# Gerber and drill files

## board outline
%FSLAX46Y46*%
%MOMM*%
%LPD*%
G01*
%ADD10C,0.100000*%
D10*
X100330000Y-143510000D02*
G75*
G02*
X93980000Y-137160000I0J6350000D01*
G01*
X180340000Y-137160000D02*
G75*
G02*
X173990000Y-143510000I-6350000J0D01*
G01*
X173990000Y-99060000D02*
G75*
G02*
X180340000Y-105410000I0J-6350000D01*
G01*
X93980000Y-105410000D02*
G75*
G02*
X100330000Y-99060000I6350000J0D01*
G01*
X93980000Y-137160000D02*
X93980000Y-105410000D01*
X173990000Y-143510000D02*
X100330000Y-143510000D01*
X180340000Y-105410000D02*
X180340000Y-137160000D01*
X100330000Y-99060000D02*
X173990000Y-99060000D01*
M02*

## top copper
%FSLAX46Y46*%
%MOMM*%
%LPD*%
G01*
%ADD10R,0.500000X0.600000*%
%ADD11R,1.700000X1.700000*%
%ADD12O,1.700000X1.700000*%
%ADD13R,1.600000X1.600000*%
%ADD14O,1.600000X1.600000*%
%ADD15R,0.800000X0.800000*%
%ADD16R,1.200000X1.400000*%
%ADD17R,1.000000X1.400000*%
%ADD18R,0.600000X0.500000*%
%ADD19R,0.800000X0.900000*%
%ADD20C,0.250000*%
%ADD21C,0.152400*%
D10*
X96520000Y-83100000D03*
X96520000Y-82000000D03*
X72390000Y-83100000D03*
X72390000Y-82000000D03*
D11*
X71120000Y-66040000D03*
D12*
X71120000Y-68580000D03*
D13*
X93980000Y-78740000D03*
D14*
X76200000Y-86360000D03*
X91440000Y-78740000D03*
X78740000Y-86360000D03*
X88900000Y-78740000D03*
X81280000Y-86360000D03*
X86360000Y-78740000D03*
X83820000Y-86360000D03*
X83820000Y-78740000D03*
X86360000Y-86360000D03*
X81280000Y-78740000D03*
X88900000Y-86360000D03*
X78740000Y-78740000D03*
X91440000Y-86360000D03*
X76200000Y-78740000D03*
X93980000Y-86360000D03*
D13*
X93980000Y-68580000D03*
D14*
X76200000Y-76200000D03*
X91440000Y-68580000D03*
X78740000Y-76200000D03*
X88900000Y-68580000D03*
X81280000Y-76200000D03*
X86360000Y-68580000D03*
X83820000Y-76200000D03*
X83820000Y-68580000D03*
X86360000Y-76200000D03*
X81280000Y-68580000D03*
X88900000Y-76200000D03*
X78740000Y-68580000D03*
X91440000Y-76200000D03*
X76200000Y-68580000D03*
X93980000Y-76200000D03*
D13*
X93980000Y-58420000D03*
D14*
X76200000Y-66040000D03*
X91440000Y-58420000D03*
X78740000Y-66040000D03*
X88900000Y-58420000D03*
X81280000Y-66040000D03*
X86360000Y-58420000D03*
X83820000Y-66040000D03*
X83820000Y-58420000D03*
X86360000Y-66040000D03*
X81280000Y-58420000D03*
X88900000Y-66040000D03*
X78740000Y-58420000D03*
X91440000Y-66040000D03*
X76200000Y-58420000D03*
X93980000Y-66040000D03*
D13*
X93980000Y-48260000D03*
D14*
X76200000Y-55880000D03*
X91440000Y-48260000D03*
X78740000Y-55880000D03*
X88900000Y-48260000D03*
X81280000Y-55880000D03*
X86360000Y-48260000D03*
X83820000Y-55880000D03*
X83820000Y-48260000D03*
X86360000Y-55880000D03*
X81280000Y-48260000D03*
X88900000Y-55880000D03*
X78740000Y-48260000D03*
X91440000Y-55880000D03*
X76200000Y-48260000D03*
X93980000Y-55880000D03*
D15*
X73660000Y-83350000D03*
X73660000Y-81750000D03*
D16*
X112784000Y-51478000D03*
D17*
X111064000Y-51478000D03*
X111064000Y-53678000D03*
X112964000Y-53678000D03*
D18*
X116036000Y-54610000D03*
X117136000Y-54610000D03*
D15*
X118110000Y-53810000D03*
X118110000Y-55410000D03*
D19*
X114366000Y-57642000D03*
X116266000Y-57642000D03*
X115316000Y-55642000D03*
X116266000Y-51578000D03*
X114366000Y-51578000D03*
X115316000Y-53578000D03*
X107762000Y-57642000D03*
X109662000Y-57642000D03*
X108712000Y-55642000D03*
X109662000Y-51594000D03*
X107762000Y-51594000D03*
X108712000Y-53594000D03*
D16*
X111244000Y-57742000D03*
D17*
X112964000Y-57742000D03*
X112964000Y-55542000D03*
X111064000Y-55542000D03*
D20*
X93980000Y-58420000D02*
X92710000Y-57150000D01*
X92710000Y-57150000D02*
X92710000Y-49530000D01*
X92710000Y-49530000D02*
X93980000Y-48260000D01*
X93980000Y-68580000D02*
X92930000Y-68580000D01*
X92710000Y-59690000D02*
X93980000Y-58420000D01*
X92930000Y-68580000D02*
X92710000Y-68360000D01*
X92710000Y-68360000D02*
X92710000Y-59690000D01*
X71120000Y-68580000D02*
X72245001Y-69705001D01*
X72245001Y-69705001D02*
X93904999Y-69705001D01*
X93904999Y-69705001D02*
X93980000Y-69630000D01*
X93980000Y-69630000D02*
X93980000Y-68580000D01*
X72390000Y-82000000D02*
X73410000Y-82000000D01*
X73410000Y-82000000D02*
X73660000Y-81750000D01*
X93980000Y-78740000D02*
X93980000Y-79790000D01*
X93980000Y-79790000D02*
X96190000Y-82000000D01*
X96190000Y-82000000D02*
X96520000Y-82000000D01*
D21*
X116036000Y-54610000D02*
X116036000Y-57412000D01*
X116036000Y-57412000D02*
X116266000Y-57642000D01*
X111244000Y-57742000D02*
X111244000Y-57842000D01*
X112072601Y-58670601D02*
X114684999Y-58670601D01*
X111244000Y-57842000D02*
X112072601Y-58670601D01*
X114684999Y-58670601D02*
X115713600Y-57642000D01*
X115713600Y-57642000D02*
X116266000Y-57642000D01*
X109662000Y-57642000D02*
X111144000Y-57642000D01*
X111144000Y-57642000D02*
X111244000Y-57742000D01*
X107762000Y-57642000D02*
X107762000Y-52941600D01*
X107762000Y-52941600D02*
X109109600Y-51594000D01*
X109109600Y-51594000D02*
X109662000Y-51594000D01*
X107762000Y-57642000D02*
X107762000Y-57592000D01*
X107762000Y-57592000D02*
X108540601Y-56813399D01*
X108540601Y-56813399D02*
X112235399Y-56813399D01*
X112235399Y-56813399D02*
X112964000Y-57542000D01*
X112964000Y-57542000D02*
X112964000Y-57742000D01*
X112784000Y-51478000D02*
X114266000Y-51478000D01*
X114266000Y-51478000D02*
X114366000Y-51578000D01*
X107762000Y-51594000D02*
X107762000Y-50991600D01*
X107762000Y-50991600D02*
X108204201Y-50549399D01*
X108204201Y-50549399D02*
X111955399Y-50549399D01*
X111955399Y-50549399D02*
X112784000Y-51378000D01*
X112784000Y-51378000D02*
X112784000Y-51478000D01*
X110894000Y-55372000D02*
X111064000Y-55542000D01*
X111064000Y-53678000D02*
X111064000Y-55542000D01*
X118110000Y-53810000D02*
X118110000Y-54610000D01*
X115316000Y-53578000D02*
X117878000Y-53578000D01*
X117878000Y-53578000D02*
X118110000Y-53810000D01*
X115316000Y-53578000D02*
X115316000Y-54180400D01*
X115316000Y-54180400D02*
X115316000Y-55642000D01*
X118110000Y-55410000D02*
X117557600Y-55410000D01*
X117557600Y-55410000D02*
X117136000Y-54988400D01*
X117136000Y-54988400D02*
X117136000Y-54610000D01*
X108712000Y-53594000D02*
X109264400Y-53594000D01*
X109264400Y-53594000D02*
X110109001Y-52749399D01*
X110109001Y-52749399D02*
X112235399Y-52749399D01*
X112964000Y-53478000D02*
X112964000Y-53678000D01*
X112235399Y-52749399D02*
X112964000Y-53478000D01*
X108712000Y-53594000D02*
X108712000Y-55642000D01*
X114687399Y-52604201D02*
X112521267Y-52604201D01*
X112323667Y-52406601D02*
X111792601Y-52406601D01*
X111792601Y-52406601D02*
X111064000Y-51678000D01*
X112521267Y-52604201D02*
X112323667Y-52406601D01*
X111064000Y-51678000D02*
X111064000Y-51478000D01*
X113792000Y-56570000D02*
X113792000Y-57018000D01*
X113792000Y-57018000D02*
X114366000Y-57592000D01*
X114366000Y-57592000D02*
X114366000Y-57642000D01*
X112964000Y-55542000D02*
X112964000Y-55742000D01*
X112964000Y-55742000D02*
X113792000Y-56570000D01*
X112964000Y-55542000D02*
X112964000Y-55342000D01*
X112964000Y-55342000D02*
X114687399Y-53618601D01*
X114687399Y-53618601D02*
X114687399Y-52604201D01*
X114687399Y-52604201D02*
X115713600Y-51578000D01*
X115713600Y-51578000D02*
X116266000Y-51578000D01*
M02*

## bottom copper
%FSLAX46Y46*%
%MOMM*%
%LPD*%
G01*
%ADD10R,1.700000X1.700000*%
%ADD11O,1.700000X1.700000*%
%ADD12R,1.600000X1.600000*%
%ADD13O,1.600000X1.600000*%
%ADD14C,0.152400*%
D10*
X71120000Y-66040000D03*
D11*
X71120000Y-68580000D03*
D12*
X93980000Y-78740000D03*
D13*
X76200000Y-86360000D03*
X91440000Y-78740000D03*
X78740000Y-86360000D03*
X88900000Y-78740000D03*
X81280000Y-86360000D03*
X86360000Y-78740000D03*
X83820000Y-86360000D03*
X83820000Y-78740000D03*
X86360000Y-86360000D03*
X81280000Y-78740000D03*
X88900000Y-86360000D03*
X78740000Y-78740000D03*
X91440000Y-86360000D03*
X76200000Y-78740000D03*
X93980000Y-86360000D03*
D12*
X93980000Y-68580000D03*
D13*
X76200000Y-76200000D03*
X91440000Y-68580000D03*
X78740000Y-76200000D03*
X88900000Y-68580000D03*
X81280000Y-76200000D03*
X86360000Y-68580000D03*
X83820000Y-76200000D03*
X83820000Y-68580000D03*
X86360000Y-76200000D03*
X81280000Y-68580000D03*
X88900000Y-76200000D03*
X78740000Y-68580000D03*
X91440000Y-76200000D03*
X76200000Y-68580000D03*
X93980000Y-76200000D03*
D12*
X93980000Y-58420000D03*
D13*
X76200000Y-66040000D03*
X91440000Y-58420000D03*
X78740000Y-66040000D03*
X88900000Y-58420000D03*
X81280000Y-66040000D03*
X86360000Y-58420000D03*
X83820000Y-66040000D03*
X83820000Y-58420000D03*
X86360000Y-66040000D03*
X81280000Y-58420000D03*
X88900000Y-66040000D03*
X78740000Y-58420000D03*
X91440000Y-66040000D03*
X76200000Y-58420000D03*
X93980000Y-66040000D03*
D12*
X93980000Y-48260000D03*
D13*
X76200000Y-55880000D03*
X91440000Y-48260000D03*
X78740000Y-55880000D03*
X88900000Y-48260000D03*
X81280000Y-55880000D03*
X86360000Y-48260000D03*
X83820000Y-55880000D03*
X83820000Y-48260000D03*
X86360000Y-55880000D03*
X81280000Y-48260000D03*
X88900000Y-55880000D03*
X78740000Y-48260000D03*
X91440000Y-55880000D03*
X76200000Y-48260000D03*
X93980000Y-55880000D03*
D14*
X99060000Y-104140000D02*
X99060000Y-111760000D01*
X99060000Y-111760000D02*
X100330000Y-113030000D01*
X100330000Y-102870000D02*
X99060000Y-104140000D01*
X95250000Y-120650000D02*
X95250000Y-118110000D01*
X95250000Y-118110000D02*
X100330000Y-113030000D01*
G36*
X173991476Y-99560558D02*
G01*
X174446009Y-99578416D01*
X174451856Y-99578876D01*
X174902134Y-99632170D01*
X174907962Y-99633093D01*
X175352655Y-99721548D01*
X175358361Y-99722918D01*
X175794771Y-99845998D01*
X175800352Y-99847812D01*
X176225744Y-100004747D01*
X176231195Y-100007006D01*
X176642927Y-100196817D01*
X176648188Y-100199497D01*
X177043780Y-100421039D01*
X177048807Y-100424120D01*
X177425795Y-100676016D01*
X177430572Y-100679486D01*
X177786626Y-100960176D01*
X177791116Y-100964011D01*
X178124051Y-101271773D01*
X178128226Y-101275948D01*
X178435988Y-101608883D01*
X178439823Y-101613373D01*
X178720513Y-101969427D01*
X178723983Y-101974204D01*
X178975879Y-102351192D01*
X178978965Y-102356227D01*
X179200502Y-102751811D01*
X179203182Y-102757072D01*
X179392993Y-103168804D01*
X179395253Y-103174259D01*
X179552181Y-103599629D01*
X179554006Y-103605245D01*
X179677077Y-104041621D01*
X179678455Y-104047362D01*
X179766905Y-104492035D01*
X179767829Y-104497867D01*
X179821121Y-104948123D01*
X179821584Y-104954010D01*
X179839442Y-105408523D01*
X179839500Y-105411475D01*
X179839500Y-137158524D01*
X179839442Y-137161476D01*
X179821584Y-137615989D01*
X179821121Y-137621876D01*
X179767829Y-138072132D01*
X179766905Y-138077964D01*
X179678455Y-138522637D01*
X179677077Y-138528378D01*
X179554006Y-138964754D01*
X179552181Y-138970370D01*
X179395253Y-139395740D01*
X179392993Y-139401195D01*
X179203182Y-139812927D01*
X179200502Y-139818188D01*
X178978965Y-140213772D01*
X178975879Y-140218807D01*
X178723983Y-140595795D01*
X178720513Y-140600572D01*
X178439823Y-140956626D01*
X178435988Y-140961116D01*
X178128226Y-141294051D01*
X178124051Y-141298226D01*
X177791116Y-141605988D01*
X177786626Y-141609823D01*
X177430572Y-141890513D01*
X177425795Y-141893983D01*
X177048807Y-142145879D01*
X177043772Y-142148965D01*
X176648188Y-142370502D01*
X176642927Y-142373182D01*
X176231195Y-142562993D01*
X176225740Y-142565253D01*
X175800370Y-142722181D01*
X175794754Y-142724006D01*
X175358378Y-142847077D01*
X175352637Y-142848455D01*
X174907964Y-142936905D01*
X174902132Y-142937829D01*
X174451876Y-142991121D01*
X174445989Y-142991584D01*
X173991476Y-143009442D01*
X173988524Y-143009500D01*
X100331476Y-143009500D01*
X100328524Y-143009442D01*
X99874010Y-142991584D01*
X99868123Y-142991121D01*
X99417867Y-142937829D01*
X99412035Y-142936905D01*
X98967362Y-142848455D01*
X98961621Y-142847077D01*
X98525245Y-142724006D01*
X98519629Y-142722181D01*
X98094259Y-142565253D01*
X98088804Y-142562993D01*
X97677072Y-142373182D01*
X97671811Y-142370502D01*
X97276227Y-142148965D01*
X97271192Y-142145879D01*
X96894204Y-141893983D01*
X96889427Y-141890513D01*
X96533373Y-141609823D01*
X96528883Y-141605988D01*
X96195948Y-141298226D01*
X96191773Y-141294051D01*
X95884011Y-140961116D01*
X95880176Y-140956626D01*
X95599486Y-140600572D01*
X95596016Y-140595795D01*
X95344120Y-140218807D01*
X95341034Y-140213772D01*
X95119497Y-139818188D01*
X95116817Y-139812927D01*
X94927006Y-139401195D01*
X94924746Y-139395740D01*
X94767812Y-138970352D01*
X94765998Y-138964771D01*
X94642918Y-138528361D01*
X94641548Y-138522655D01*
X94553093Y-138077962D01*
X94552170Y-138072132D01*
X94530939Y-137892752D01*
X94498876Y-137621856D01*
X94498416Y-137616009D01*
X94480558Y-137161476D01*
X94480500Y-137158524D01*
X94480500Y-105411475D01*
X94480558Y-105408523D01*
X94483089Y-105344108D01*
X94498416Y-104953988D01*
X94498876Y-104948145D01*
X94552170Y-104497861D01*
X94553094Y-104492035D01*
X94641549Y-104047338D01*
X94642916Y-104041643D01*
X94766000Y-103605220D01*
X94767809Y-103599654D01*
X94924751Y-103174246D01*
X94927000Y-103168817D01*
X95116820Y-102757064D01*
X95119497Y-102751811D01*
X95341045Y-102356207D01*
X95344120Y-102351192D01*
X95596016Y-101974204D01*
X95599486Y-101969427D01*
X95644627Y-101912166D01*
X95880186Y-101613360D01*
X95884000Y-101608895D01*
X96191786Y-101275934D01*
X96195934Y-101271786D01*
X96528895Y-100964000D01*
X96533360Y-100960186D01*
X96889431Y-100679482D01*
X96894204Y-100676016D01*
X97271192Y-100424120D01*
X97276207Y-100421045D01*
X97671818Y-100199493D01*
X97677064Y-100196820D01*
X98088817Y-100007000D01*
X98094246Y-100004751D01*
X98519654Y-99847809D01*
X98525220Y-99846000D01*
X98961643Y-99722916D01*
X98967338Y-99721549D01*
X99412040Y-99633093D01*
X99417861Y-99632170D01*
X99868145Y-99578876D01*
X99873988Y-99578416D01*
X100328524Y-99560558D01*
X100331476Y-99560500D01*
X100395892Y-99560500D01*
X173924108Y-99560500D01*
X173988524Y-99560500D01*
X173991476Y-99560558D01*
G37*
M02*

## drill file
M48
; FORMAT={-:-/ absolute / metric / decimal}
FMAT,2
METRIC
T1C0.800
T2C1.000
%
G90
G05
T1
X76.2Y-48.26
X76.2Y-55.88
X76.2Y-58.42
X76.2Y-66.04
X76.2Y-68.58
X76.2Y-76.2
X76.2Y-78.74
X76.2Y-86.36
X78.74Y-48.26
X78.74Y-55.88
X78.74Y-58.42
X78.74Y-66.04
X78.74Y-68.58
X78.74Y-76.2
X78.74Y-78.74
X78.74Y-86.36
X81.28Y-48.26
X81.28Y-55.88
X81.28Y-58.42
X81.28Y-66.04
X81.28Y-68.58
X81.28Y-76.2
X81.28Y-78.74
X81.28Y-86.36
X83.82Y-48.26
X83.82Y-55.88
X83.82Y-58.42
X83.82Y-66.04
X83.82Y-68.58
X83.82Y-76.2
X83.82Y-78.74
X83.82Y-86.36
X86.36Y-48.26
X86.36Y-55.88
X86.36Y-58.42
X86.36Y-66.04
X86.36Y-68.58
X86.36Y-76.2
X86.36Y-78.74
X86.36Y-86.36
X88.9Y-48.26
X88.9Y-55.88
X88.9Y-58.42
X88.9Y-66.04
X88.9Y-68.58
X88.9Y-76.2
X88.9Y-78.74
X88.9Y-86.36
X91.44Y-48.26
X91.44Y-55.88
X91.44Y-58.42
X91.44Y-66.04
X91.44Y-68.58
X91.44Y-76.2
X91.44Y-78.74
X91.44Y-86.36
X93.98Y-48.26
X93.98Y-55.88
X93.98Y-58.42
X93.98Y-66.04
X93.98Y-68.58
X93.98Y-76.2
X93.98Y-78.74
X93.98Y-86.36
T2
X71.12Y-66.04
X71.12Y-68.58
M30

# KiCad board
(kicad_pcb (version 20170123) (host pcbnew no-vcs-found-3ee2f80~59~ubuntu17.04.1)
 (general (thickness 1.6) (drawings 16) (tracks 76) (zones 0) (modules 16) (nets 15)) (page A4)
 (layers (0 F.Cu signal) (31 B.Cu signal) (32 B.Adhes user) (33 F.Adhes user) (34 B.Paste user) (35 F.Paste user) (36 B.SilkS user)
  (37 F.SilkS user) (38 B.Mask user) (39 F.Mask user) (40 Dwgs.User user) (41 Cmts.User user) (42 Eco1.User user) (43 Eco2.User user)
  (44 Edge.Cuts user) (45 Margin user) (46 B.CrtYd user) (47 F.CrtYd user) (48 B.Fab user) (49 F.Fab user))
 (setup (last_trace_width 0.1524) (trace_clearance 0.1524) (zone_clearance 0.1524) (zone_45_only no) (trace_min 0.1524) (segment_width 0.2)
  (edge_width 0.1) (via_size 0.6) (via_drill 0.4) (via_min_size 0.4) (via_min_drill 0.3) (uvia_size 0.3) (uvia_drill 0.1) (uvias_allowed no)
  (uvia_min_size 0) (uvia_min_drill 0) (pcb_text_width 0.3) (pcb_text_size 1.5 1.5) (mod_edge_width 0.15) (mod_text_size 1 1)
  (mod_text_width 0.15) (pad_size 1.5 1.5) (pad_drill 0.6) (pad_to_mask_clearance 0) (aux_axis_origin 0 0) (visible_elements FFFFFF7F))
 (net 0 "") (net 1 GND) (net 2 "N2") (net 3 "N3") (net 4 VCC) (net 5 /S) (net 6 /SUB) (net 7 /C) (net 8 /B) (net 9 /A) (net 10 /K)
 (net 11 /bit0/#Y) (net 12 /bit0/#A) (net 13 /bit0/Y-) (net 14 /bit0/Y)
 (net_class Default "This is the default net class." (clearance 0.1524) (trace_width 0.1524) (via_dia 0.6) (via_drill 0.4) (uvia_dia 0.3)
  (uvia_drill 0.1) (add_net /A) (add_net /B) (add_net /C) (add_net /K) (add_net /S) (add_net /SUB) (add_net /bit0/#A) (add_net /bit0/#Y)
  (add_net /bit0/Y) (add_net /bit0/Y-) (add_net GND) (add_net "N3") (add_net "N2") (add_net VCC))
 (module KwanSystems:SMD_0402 (layer F.Cu) (at 96.52 82.55 270)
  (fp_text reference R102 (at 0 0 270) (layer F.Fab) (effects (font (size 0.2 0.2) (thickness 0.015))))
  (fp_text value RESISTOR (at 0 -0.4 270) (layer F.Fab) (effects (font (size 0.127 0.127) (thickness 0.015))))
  (pad 2 smd rect (at 0.55 0 270) (size 0.6 0.5) (layers F.Cu F.Paste F.Mask) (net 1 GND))
  (pad 1 smd rect (at -0.55 0 270) (size 0.6 0.5) (layers F.Cu F.Paste F.Mask) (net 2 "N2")))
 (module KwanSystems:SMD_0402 (layer F.Cu) (at 72.39 82.55 270)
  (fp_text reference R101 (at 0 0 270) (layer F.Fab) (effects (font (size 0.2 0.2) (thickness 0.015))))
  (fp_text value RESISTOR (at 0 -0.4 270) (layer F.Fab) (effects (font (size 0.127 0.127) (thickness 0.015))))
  (pad 2 smd rect (at 0.55 0 270) (size 0.6 0.5) (layers F.Cu F.Paste F.Mask) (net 1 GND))
  (pad 1 smd rect (at -0.55 0 270) (size 0.6 0.5) (layers F.Cu F.Paste F.Mask) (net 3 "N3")))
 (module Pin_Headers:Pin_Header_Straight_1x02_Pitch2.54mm (layer F.Cu) (at 71.12 66.04)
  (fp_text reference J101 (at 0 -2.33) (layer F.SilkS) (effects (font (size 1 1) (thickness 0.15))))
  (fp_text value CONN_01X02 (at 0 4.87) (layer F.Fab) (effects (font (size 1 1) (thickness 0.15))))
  (pad 1 thru_hole rect (at 0 0) (size 1.7 1.7) (drill 1) (layers *.Cu *.Mask) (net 1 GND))
  (pad 2 thru_hole oval (at 0 2.54) (size 1.7 1.7) (drill 1) (layers *.Cu *.Mask) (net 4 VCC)))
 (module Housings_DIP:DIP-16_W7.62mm (layer F.Cu) (at 93.98 78.74 270)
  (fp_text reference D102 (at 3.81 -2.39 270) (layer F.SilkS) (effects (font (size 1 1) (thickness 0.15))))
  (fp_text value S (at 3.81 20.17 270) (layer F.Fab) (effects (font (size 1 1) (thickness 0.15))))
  (pad 1 thru_hole rect (at 0 0 270) (size 1.6 1.6) (drill 0.8) (layers *.Cu *.Mask) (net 2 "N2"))
  (pad 9 thru_hole oval (at 7.62 17.78 270) (size 1.6 1.6) (drill 0.8) (layers *.Cu *.Mask))
  (pad 2 thru_hole oval (at 0 2.54 270) (size 1.6 1.6) (drill 0.8) (layers *.Cu *.Mask))
  (pad 10 thru_hole oval (at 7.62 15.24 270) (size 1.6 1.6) (drill 0.8) (layers *.Cu *.Mask))
  (pad 3 thru_hole oval (at 0 5.08 270) (size 1.6 1.6) (drill 0.8) (layers *.Cu *.Mask))
  (pad 11 thru_hole oval (at 7.62 12.7 270) (size 1.6 1.6) (drill 0.8) (layers *.Cu *.Mask))
  (pad 4 thru_hole oval (at 0 7.62 270) (size 1.6 1.6) (drill 0.8) (layers *.Cu *.Mask))
  (pad 12 thru_hole oval (at 7.62 10.16 270) (size 1.6 1.6) (drill 0.8) (layers *.Cu *.Mask))
  (pad 5 thru_hole oval (at 0 10.16 270) (size 1.6 1.6) (drill 0.8) (layers *.Cu *.Mask))
  (pad 13 thru_hole oval (at 7.62 7.62 270) (size 1.6 1.6) (drill 0.8) (layers *.Cu *.Mask))
  (pad 6 thru_hole oval (at 0 12.7 270) (size 1.6 1.6) (drill 0.8) (layers *.Cu *.Mask))
  (pad 14 thru_hole oval (at 7.62 5.08 270) (size 1.6 1.6) (drill 0.8) (layers *.Cu *.Mask))
  (pad 7 thru_hole oval (at 0 15.24 270) (size 1.6 1.6) (drill 0.8) (layers *.Cu *.Mask))
  (pad 15 thru_hole oval (at 7.62 2.54 270) (size 1.6 1.6) (drill 0.8) (layers *.Cu *.Mask))
  (pad 8 thru_hole oval (at 0 17.78 270) (size 1.6 1.6) (drill 0.8) (layers *.Cu *.Mask))
  (pad 16 thru_hole oval (at 7.62 0 270) (size 1.6 1.6) (drill 0.8) (layers *.Cu *.Mask) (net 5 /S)))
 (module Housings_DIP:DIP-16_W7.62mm (layer F.Cu) (at 93.98 68.58 270)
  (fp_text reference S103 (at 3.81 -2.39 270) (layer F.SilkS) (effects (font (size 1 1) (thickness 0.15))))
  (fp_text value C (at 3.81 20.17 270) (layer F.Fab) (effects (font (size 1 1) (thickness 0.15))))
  (pad 1 thru_hole rect (at 0 0 270) (size 1.6 1.6) (drill 0.8) (layers *.Cu *.Mask) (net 4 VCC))
  (pad 9 thru_hole oval (at 7.62 17.78 270) (size 1.6 1.6) (drill 0.8) (layers *.Cu *.Mask))
  (pad 2 thru_hole oval (at 0 2.54 270) (size 1.6 1.6) (drill 0.8) (layers *.Cu *.Mask))
  (pad 10 thru_hole oval (at 7.62 15.24 270) (size 1.6 1.6) (drill 0.8) (layers *.Cu *.Mask))
  (pad 3 thru_hole oval (at 0 5.08 270) (size 1.6 1.6) (drill 0.8) (layers *.Cu *.Mask))
  (pad 11 thru_hole oval (at 7.62 12.7 270) (size 1.6 1.6) (drill 0.8) (layers *.Cu *.Mask))
  (pad 4 thru_hole oval (at 0 7.62 270) (size 1.6 1.6) (drill 0.8) (layers *.Cu *.Mask))
  (pad 12 thru_hole oval (at 7.62 10.16 270) (size 1.6 1.6) (drill 0.8) (layers *.Cu *.Mask))
  (pad 5 thru_hole oval (at 0 10.16 270) (size 1.6 1.6) (drill 0.8) (layers *.Cu *.Mask))
  (pad 13 thru_hole oval (at 7.62 7.62 270) (size 1.6 1.6) (drill 0.8) (layers *.Cu *.Mask))
  (pad 6 thru_hole oval (at 0 12.7 270) (size 1.6 1.6) (drill 0.8) (layers *.Cu *.Mask))
  (pad 14 thru_hole oval (at 7.62 5.08 270) (size 1.6 1.6) (drill 0.8) (layers *.Cu *.Mask))
  (pad 7 thru_hole oval (at 0 15.24 270) (size 1.6 1.6) (drill 0.8) (layers *.Cu *.Mask))
  (pad 15 thru_hole oval (at 7.62 2.54 270) (size 1.6 1.6) (drill 0.8) (layers *.Cu *.Mask) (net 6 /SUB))
  (pad 8 thru_hole oval (at 0 17.78 270) (size 1.6 1.6) (drill 0.8) (layers *.Cu *.Mask) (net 1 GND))
  (pad 16 thru_hole oval (at 7.62 0 270) (size 1.6 1.6) (drill 0.8) (layers *.Cu *.Mask) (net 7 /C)))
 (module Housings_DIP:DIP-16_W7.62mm (layer F.Cu) (at 93.98 58.42 270)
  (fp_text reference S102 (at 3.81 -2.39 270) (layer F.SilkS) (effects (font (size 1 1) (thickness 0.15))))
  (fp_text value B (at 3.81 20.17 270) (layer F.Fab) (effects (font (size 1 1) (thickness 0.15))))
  (pad 1 thru_hole rect (at 0 0 270) (size 1.6 1.6) (drill 0.8) (layers *.Cu *.Mask) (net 4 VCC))
  (pad 9 thru_hole oval (at 7.62 17.78 270) (size 1.6 1.6) (drill 0.8) (layers *.Cu *.Mask))
  (pad 2 thru_hole oval (at 0 2.54 270) (size 1.6 1.6) (drill 0.8) (layers *.Cu *.Mask))
  (pad 10 thru_hole oval (at 7.62 15.24 270) (size 1.6 1.6) (drill 0.8) (layers *.Cu *.Mask))
  (pad 3 thru_hole oval (at 0 5.08 270) (size 1.6 1.6) (drill 0.8) (layers *.Cu *.Mask))
  (pad 11 thru_hole oval (at 7.62 12.7 270) (size 1.6 1.6) (drill 0.8) (layers *.Cu *.Mask))
  (pad 4 thru_hole oval (at 0 7.62 270) (size 1.6 1.6) (drill 0.8) (layers *.Cu *.Mask))
  (pad 12 thru_hole oval (at 7.62 10.16 270) (size 1.6 1.6) (drill 0.8) (layers *.Cu *.Mask))
  (pad 5 thru_hole oval (at 0 10.16 270) (size 1.6 1.6) (drill 0.8) (layers *.Cu *.Mask))
  (pad 13 thru_hole oval (at 7.62 7.62 270) (size 1.6 1.6) (drill 0.8) (layers *.Cu *.Mask))
  (pad 6 thru_hole oval (at 0 12.7 270) (size 1.6 1.6) (drill 0.8) (layers *.Cu *.Mask))
  (pad 14 thru_hole oval (at 7.62 5.08 270) (size 1.6 1.6) (drill 0.8) (layers *.Cu *.Mask))
  (pad 7 thru_hole oval (at 0 15.24 270) (size 1.6 1.6) (drill 0.8) (layers *.Cu *.Mask))
  (pad 15 thru_hole oval (at 7.62 2.54 270) (size 1.6 1.6) (drill 0.8) (layers *.Cu *.Mask))
  (pad 8 thru_hole oval (at 0 17.78 270) (size 1.6 1.6) (drill 0.8) (layers *.Cu *.Mask) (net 1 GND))
  (pad 16 thru_hole oval (at 7.62 0 270) (size 1.6 1.6) (drill 0.8) (layers *.Cu *.Mask) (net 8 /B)))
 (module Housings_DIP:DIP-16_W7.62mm (layer F.Cu) (at 93.98 48.26 270)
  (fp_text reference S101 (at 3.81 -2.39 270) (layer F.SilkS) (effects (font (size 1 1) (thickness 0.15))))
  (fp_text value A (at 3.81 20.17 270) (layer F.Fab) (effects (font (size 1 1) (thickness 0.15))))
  (pad 1 thru_hole rect (at 0 0 270) (size 1.6 1.6) (drill 0.8) (layers *.Cu *.Mask) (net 4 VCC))
  (pad 9 thru_hole oval (at 7.62 17.78 270) (size 1.6 1.6) (drill 0.8) (layers *.Cu *.Mask))
  (pad 2 thru_hole oval (at 0 2.54 270) (size 1.6 1.6) (drill 0.8) (layers *.Cu *.Mask))
  (pad 10 thru_hole oval (at 7.62 15.24 270) (size 1.6 1.6) (drill 0.8) (layers *.Cu *.Mask))
  (pad 3 thru_hole oval (at 0 5.08 270) (size 1.6 1.6) (drill 0.8) (layers *.Cu *.Mask))
  (pad 11 thru_hole oval (at 7.62 12.7 270) (size 1.6 1.6) (drill 0.8) (layers *.Cu *.Mask))
  (pad 4 thru_hole oval (at 0 7.62 270) (size 1.6 1.6) (drill 0.8) (layers *.Cu *.Mask))
  (pad 12 thru_hole oval (at 7.62 10.16 270) (size 1.6 1.6) (drill 0.8) (layers *.Cu *.Mask))
  (pad 5 thru_hole oval (at 0 10.16 270) (size 1.6 1.6) (drill 0.8) (layers *.Cu *.Mask))
  (pad 13 thru_hole oval (at 7.62 7.62 270) (size 1.6 1.6) (drill 0.8) (layers *.Cu *.Mask))
  (pad 6 thru_hole oval (at 0 12.7 270) (size 1.6 1.6) (drill 0.8) (layers *.Cu *.Mask))
  (pad 14 thru_hole oval (at 7.62 5.08 270) (size 1.6 1.6) (drill 0.8) (layers *.Cu *.Mask))
  (pad 7 thru_hole oval (at 0 15.24 270) (size 1.6 1.6) (drill 0.8) (layers *.Cu *.Mask))
  (pad 15 thru_hole oval (at 7.62 2.54 270) (size 1.6 1.6) (drill 0.8) (layers *.Cu *.Mask))
  (pad 8 thru_hole oval (at 0 17.78 270) (size 1.6 1.6) (drill 0.8) (layers *.Cu *.Mask) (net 1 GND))
  (pad 16 thru_hole oval (at 7.62 0 270) (size 1.6 1.6) (drill 0.8) (layers *.Cu *.Mask) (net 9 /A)))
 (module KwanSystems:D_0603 (layer F.Cu) (at 73.66 82.55 270)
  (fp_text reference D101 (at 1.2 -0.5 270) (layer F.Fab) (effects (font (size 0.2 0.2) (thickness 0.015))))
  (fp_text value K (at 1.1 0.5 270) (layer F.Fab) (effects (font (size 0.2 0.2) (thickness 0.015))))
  (pad 2 smd rect (at 0.8 0 90) (size 0.8 0.8) (layers F.Cu F.Paste F.Mask) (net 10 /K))
  (pad 1 smd rect (at -0.8 0 90) (size 0.8 0.8) (layers F.Cu F.Paste F.Mask) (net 3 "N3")))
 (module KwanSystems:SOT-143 (layer F.Cu) (at 112.014 52.578 270)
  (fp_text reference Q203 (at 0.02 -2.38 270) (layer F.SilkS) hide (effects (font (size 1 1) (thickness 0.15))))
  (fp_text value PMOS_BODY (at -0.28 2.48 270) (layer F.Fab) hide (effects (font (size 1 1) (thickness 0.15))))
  (pad 1 smd rect (at -1.1 -0.77 180) (size 1.2 1.4) (layers F.Cu F.Paste F.Mask) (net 4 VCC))
  (pad 2 smd rect (at -1.1 0.95 180) (size 1 1.4) (layers F.Cu F.Paste F.Mask) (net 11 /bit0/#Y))
  (pad 3 smd rect (at 1.1 0.95 180) (size 1 1.4) (layers F.Cu F.Paste F.Mask) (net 8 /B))
  (pad 4 smd rect (at 1.1 -0.95 180) (size 1 1.4) (layers F.Cu F.Paste F.Mask) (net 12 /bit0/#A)))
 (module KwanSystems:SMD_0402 (layer F.Cu) (at 116.586 54.61 180)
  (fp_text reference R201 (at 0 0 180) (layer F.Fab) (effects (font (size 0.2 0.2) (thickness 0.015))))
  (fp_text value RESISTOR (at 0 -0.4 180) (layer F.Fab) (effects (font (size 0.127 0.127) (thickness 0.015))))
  (pad 2 smd rect (at 0.55 0 180) (size 0.6 0.5) (layers F.Cu F.Paste F.Mask) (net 1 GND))
  (pad 1 smd rect (at -0.55 0 180) (size 0.6 0.5) (layers F.Cu F.Paste F.Mask) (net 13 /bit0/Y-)))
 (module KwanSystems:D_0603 (layer F.Cu) (at 118.11 54.61 90)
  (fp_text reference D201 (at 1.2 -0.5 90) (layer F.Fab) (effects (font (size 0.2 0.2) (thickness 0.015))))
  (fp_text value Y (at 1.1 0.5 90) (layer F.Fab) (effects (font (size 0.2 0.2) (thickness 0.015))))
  (pad 2 smd rect (at 0.8 0 270) (size 0.8 0.8) (layers F.Cu F.Paste F.Mask) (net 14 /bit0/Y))
  (pad 1 smd rect (at -0.8 0 270) (size 0.8 0.8) (layers F.Cu F.Paste F.Mask) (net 13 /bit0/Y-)))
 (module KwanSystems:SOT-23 (layer F.Cu) (at 115.316 56.642 90)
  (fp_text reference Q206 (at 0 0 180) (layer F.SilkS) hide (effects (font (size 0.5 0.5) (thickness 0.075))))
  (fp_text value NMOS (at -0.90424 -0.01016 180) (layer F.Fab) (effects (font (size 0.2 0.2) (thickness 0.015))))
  (pad 1 smd rect (at -1 -0.95 90) (size 0.9 0.8) (layers F.Cu F.Paste F.Mask) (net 11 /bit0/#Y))
  (pad 2 smd rect (at -1 0.95 90) (size 0.9 0.8) (layers F.Cu F.Paste F.Mask) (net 1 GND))
  (pad 3 smd rect (at 1 0 90) (size 0.9 0.8) (layers F.Cu F.Paste F.Mask) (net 14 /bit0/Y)))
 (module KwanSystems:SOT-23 (layer F.Cu) (at 115.316 52.578 270)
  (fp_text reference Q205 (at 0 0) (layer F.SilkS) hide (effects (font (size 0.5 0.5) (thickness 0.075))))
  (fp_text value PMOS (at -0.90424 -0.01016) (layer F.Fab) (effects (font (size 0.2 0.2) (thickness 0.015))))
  (pad 1 smd rect (at -1 -0.95 270) (size 0.9 0.8) (layers F.Cu F.Paste F.Mask) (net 11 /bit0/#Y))
  (pad 2 smd rect (at -1 0.95 270) (size 0.9 0.8) (layers F.Cu F.Paste F.Mask) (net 4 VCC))
  (pad 3 smd rect (at 1 0 270) (size 0.9 0.8) (layers F.Cu F.Paste F.Mask) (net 14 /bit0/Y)))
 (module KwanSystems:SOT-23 (layer F.Cu) (at 108.712 56.642 90)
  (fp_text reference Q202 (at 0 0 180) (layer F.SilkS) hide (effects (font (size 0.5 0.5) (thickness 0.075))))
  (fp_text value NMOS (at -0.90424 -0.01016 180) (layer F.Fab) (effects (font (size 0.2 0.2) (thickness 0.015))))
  (pad 1 smd rect (at -1 -0.95 90) (size 0.9 0.8) (layers F.Cu F.Paste F.Mask) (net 9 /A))
  (pad 2 smd rect (at -1 0.95 90) (size 0.9 0.8) (layers F.Cu F.Paste F.Mask) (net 1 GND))
  (pad 3 smd rect (at 1 0 90) (size 0.9 0.8) (layers F.Cu F.Paste F.Mask) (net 12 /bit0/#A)))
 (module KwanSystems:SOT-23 (layer F.Cu) (at 108.712 52.594 270)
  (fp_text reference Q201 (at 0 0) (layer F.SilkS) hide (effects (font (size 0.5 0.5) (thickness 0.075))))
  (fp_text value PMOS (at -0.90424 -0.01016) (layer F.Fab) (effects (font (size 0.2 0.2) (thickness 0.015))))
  (pad 1 smd rect (at -1 -0.95 270) (size 0.9 0.8) (layers F.Cu F.Paste F.Mask) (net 9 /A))
  (pad 2 smd rect (at -1 0.95 270) (size 0.9 0.8) (layers F.Cu F.Paste F.Mask) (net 4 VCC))
  (pad 3 smd rect (at 1 0 270) (size 0.9 0.8) (layers F.Cu F.Paste F.Mask) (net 12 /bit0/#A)))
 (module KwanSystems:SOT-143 (layer F.Cu) (at 112.014 56.642 90)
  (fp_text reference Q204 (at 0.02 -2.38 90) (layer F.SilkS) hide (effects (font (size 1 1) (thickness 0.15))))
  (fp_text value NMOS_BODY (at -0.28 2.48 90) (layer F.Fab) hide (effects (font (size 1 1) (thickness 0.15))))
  (pad 1 smd rect (at -1.1 -0.77) (size 1.2 1.4) (layers F.Cu F.Paste F.Mask) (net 1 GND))
  (pad 2 smd rect (at -1.1 0.95) (size 1 1.4) (layers F.Cu F.Paste F.Mask) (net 9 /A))
  (pad 3 smd rect (at 1.1 0.95) (size 1 1.4) (layers F.Cu F.Paste F.Mask) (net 11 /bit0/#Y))
  (pad 4 smd rect (at 1.1 -0.95) (size 1 1.4) (layers F.Cu F.Paste F.Mask) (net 8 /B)))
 (gr_arc (start 100.33 137.16) (end 100.33 143.51) (angle 90) (layer Edge.Cuts) (width 0.1))
 (gr_arc (start 173.99 137.16) (end 180.34 137.16) (angle 90) (layer Edge.Cuts) (width 0.1))
 (gr_arc (start 173.99 105.41) (end 173.99 99.06) (angle 90) (layer Edge.Cuts) (width 0.1))
 (gr_arc (start 100.33 105.41) (end 93.98 105.41) (angle 90) (layer Edge.Cuts) (width 0.1))
 (gr_line (start 93.98 137.16) (end 93.98 105.41) (layer Edge.Cuts) (width 0.1))
 (gr_line (start 173.99 143.51) (end 100.33 143.51) (layer Edge.Cuts) (width 0.1))
 (gr_line (start 180.34 105.41) (end 180.34 137.16) (layer Edge.Cuts) (width 0.1))
 (gr_line (start 100.33 99.06) (end 173.99 99.06) (layer Edge.Cuts) (width 0.1))
 (segment (start 93.98 58.42) (end 92.71 57.15) (width 0.25) (layer F.Cu) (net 4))
 (segment (start 92.71 57.15) (end 92.71 49.53) (width 0.25) (layer F.Cu) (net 4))
 (segment (start 92.71 49.53) (end 93.98 48.26) (width 0.25) (layer F.Cu) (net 4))
 (segment (start 93.98 68.58) (end 92.93 68.58) (width 0.25) (layer F.Cu) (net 4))
 (segment (start 92.71 59.69) (end 93.98 58.42) (width 0.25) (layer F.Cu) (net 4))
 (segment (start 92.93 68.58) (end 92.71 68.36) (width 0.25) (layer F.Cu) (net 4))
 (segment (start 92.71 68.36) (end 92.71 59.69) (width 0.25) (layer F.Cu) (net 4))
 (segment (start 71.12 68.58) (end 72.245001 69.705001) (width 0.25) (layer F.Cu) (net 4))
 (segment (start 72.245001 69.705001) (end 93.904999 69.705001) (width 0.25) (layer F.Cu) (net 4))
 (segment (start 93.904999 69.705001) (end 93.98 69.63) (width 0.25) (layer F.Cu) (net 4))
 (segment (start 93.98 69.63) (end 93.98 68.58) (width 0.25) (layer F.Cu) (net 4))
 (segment (start 72.39 82) (end 73.41 82) (width 0.25) (layer F.Cu) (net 3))
 (segment (start 73.41 82) (end 73.66 81.75) (width 0.25) (layer F.Cu) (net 3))
 (segment (start 93.98 78.74) (end 93.98 79.79) (width 0.25) (layer F.Cu) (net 2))
 (segment (start 93.98 79.79) (end 96.19 82) (width 0.25) (layer F.Cu) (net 2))
 (segment (start 96.19 82) (end 96.52 82) (width 0.25) (layer F.Cu) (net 2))
 (segment (start 99.06 104.14) (end 99.06 111.76) (width 0.1524) (layer B.Cu) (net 1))
 (segment (start 99.06 111.76) (end 100.33 113.03) (width 0.1524) (layer B.Cu) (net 1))
 (segment (start 100.33 102.87) (end 99.06 104.14) (width 0.1524) (layer B.Cu) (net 1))
 (segment (start 95.25 120.65) (end 95.25 118.11) (width 0.1524) (layer B.Cu) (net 1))
 (segment (start 95.25 118.11) (end 100.33 113.03) (width 0.1524) (layer B.Cu) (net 1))
 (segment (start 116.036 54.61) (end 116.036 57.412) (width 0.1524) (layer F.Cu) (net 1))
 (segment (start 116.036 57.412) (end 116.266 57.642) (width 0.1524) (layer F.Cu) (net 1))
 (segment (start 111.244 57.742) (end 111.244 57.842) (width 0.1524) (layer F.Cu) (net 1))
 (segment (start 112.072601 58.670601) (end 114.684999 58.670601) (width 0.1524) (layer F.Cu) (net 1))
 (segment (start 111.244 57.842) (end 112.072601 58.670601) (width 0.1524) (layer F.Cu) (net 1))
 (segment (start 114.684999 58.670601) (end 115.7136 57.642) (width 0.1524) (layer F.Cu) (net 1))
 (segment (start 115.7136 57.642) (end 116.266 57.642) (width 0.1524) (layer F.Cu) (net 1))
 (segment (start 109.662 57.642) (end 111.144 57.642) (width 0.1524) (layer F.Cu) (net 1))
 (segment (start 111.144 57.642) (end 111.244 57.742) (width 0.1524) (layer F.Cu) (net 1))
 (segment (start 107.762 57.642) (end 107.762 52.9416) (width 0.1524) (layer F.Cu) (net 9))
 (segment (start 107.762 52.9416) (end 109.1096 51.594) (width 0.1524) (layer F.Cu) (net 9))
 (segment (start 109.1096 51.594) (end 109.662 51.594) (width 0.1524) (layer F.Cu) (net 9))
 (segment (start 107.762 57.642) (end 107.762 57.592) (width 0.1524) (layer F.Cu) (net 9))
 (segment (start 107.762 57.592) (end 108.540601 56.813399) (width 0.1524) (layer F.Cu) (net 9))
 (segment (start 108.540601 56.813399) (end 112.235399 56.813399) (width 0.1524) (layer F.Cu) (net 9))
 (segment (start 112.235399 56.813399) (end 112.964 57.542) (width 0.1524) (layer F.Cu) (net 9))
 (segment (start 112.964 57.542) (end 112.964 57.742) (width 0.1524) (layer F.Cu) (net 9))
 (segment (start 112.784 51.478) (end 114.266 51.478) (width 0.1524) (layer F.Cu) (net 4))
 (segment (start 114.266 51.478) (end 114.366 51.578) (width 0.1524) (layer F.Cu) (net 4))
 (segment (start 107.762 51.594) (end 107.762 50.9916) (width 0.1524) (layer F.Cu) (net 4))
 (segment (start 107.762 50.9916) (end 108.204201 50.549399) (width 0.1524) (layer F.Cu) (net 4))
 (segment (start 108.204201 50.549399) (end 111.955399 50.549399) (width 0.1524) (layer F.Cu) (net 4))
 (segment (start 111.955399 50.549399) (end 112.784 51.378) (width 0.1524) (layer F.Cu) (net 4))
 (segment (start 112.784 51.378) (end 112.784 51.478) (width 0.1524) (layer F.Cu) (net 4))
 (segment (start 110.894 55.372) (end 111.064 55.542) (width 0.1524) (layer F.Cu) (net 8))
 (segment (start 111.064 53.678) (end 111.064 55.542) (width 0.1524) (layer F.Cu) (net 8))
 (segment (start 118.11 53.81) (end 118.11 54.61) (width 0.1524) (layer F.Cu) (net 14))
 (segment (start 115.316 53.578) (end 117.878 53.578) (width 0.1524) (layer F.Cu) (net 14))
 (segment (start 117.878 53.578) (end 118.11 53.81) (width 0.1524) (layer F.Cu) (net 14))
 (segment (start 115.316 53.578) (end 115.316 54.1804) (width 0.1524) (layer F.Cu) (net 14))
 (segment (start 115.316 54.1804) (end 115.316 55.642) (width 0.1524) (layer F.Cu) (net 14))
 (segment (start 118.11 55.41) (end 117.5576 55.41) (width 0.1524) (layer F.Cu) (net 13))
 (segment (start 117.5576 55.41) (end 117.136 54.9884) (width 0.1524) (layer F.Cu) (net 13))
 (segment (start 117.136 54.9884) (end 117.136 54.61) (width 0.1524) (layer F.Cu) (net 13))
 (segment (start 108.712 53.594) (end 109.2644 53.594) (width 0.1524) (layer F.Cu) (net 12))
 (segment (start 109.2644 53.594) (end 110.109001 52.749399) (width 0.1524) (layer F.Cu) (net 12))
 (segment (start 110.109001 52.749399) (end 112.235399 52.749399) (width 0.1524) (layer F.Cu) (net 12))
 (segment (start 112.964 53.478) (end 112.964 53.678) (width 0.1524) (layer F.Cu) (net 12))
 (segment (start 112.235399 52.749399) (end 112.964 53.478) (width 0.1524) (layer F.Cu) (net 12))
 (segment (start 108.712 53.594) (end 108.712 55.642) (width 0.1524) (layer F.Cu) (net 12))
 (segment (start 114.687399 52.604201) (end 112.521267 52.604201) (width 0.1524) (layer F.Cu) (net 11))
 (segment (start 112.323667 52.406601) (end 111.792601 52.406601) (width 0.1524) (layer F.Cu) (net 11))
 (segment (start 111.792601 52.406601) (end 111.064 51.678) (width 0.1524) (layer F.Cu) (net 11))
 (segment (start 112.521267 52.604201) (end 112.323667 52.406601) (width 0.1524) (layer F.Cu) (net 11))
 (segment (start 111.064 51.678) (end 111.064 51.478) (width 0.1524) (layer F.Cu) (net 11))
 (segment (start 113.792 56.57) (end 113.792 57.018) (width 0.1524) (layer F.Cu) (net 11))
 (segment (start 113.792 57.018) (end 114.366 57.592) (width 0.1524) (layer F.Cu) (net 11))
 (segment (start 114.366 57.592) (end 114.366 57.642) (width 0.1524) (layer F.Cu) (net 11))
 (segment (start 112.964 55.542) (end 112.964 55.742) (width 0.1524) (layer F.Cu) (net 11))
 (segment (start 112.964 55.742) (end 113.792 56.57) (width 0.1524) (layer F.Cu) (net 11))
 (segment (start 112.964 55.542) (end 112.964 55.342) (width 0.1524) (layer F.Cu) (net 11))
 (segment (start 112.964 55.342) (end 114.687399 53.618601) (width 0.1524) (layer F.Cu) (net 11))
 (segment (start 114.687399 53.618601) (end 114.687399 52.604201) (width 0.1524) (layer F.Cu) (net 11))
 (segment (start 114.687399 52.604201) (end 115.7136 51.578) (width 0.1524) (layer F.Cu) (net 11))
 (segment (start 115.7136 51.578) (end 116.266 51.578) (width 0.1524) (layer F.Cu) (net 11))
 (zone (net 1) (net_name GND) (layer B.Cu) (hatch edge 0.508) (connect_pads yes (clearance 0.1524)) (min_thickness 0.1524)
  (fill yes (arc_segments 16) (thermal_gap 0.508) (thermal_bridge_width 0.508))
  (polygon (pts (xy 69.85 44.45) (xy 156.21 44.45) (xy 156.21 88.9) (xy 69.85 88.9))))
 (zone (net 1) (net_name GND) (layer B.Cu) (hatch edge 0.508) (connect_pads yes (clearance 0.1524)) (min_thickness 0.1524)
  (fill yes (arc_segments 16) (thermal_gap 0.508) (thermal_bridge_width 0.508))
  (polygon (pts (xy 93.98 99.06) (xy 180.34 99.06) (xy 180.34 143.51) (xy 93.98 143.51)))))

